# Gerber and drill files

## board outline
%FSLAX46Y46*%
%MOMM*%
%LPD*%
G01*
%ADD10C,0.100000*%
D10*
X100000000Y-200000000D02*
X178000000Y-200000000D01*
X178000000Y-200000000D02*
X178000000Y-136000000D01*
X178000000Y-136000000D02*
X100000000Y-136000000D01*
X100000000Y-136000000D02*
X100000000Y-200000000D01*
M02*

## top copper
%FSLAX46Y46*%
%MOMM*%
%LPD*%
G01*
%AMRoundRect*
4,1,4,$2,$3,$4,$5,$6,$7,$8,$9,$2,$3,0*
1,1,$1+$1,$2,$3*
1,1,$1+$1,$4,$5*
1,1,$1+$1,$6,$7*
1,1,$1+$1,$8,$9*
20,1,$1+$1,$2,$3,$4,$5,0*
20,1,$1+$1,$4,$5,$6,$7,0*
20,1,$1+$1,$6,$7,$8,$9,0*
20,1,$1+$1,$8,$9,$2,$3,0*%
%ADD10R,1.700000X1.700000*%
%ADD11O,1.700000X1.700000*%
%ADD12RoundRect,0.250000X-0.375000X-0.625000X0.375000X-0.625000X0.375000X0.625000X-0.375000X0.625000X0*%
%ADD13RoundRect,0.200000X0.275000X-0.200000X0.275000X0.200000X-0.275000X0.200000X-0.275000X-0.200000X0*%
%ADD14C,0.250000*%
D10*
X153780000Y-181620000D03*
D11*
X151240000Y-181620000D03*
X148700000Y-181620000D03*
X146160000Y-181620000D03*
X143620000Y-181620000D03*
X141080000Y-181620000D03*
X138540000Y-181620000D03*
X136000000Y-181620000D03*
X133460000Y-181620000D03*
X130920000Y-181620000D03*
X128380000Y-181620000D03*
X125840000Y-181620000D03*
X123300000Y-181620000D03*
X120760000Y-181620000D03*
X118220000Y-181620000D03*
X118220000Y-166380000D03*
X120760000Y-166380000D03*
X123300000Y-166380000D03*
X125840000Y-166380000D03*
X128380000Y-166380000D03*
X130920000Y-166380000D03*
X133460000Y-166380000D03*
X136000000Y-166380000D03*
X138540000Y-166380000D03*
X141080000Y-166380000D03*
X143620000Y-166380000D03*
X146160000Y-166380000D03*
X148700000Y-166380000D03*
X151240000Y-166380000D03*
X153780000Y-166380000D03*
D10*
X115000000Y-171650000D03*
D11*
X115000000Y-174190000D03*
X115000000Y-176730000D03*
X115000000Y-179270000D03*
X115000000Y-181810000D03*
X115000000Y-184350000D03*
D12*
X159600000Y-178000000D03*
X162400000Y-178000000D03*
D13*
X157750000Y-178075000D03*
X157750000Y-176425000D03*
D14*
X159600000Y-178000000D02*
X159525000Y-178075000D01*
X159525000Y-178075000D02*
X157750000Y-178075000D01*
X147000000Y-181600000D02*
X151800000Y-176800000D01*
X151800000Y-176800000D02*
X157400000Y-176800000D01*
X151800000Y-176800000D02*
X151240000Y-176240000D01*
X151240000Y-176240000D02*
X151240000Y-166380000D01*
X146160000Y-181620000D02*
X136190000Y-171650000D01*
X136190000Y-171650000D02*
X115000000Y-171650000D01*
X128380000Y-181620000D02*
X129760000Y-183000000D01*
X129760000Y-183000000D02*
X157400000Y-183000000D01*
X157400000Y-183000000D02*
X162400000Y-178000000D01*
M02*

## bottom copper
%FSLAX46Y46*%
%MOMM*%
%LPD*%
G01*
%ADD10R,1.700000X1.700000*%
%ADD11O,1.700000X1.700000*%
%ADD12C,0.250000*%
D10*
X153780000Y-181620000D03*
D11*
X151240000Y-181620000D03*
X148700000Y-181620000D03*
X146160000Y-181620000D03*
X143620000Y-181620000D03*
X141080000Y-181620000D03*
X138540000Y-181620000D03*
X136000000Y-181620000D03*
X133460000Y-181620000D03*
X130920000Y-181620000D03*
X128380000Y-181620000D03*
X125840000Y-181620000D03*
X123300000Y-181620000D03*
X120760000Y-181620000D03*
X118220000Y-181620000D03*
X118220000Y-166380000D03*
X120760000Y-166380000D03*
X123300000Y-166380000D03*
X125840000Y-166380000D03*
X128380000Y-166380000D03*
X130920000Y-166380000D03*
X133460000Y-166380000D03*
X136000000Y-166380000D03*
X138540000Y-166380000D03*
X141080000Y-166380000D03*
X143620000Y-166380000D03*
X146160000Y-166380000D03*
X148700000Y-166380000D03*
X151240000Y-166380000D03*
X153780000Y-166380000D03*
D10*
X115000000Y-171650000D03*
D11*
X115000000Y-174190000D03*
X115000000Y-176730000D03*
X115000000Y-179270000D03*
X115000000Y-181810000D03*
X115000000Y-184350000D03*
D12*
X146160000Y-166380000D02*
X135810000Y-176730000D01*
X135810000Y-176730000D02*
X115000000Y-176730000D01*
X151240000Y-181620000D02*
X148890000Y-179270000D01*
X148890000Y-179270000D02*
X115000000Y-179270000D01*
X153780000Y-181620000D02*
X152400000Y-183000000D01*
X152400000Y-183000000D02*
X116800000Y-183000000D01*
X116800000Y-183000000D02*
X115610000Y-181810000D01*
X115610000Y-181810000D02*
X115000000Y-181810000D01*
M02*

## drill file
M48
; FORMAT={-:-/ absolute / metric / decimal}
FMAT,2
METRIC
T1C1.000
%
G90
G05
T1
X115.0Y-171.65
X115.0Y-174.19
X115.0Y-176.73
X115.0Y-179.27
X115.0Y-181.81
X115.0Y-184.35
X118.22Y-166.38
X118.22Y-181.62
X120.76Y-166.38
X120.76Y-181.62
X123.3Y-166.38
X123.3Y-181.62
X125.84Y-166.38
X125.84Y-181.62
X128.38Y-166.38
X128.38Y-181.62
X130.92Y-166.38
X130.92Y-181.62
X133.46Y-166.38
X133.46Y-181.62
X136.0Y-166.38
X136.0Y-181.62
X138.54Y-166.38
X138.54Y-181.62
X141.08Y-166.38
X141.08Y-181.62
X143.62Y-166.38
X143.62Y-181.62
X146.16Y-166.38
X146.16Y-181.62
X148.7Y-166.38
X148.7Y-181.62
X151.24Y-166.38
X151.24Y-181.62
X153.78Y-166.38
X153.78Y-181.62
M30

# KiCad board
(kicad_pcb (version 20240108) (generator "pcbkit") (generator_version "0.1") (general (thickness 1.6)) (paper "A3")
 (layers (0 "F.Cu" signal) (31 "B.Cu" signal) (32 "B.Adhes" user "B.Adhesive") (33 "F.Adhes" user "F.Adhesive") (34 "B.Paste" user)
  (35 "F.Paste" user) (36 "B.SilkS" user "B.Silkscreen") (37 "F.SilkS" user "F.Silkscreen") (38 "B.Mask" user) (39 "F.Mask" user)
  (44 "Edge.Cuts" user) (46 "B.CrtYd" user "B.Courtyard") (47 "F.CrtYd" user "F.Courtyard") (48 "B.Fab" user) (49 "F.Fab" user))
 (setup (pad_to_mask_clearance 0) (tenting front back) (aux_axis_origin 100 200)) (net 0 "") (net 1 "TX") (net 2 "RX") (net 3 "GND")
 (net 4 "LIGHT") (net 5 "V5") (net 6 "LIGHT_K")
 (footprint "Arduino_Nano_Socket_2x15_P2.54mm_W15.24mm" (layer "B.Cu") (at 136 174 90)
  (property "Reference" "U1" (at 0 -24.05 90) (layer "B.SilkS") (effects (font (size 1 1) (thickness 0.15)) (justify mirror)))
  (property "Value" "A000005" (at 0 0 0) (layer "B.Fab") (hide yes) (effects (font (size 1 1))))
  (pad "1" thru_hole rect (at -7.62 17.78 90) (size 1.7 1.7) (drill 1) (layers "*.Cu" "*.Mask") (solder_mask_margin 0.05) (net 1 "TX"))
  (pad "2" thru_hole oval (at -7.62 15.24 90) (size 1.7 1.7) (drill 1) (layers "*.Cu" "*.Mask") (solder_mask_margin 0.05) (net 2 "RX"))
  (pad "3" thru_hole oval (at -7.62 12.7 90) (size 1.7 1.7) (drill 1) (layers "*.Cu" "*.Mask") (solder_mask_margin 0.05))
  (pad "4" thru_hole oval (at -7.62 10.16 90) (size 1.7 1.7) (drill 1) (layers "*.Cu" "*.Mask") (solder_mask_margin 0.05) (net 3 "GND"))
  (pad "5" thru_hole oval (at -7.62 7.62 90) (size 1.7 1.7) (drill 1) (layers "*.Cu" "*.Mask") (solder_mask_margin 0.05))
  (pad "6" thru_hole oval (at -7.62 5.08 90) (size 1.7 1.7) (drill 1) (layers "*.Cu" "*.Mask") (solder_mask_margin 0.05))
  (pad "7" thru_hole oval (at -7.62 2.54 90) (size 1.7 1.7) (drill 1) (layers "*.Cu" "*.Mask") (solder_mask_margin 0.05))
  (pad "8" thru_hole oval (at -7.62 0 90) (size 1.7 1.7) (drill 1) (layers "*.Cu" "*.Mask") (solder_mask_margin 0.05))
  (pad "9" thru_hole oval (at -7.62 -2.54 90) (size 1.7 1.7) (drill 1) (layers "*.Cu" "*.Mask") (solder_mask_margin 0.05))
  (pad "10" thru_hole oval (at -7.62 -5.08 90) (size 1.7 1.7) (drill 1) (layers "*.Cu" "*.Mask") (solder_mask_margin 0.05))
  (pad "11" thru_hole oval (at -7.62 -7.62 90) (size 1.7 1.7) (drill 1) (layers "*.Cu" "*.Mask") (solder_mask_margin 0.05) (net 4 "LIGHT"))
  (pad "12" thru_hole oval (at -7.62 -10.16 90) (size 1.7 1.7) (drill 1) (layers "*.Cu" "*.Mask") (solder_mask_margin 0.05))
  (pad "13" thru_hole oval (at -7.62 -12.7 90) (size 1.7 1.7) (drill 1) (layers "*.Cu" "*.Mask") (solder_mask_margin 0.05))
  (pad "14" thru_hole oval (at -7.62 -15.24 90) (size 1.7 1.7) (drill 1) (layers "*.Cu" "*.Mask") (solder_mask_margin 0.05))
  (pad "15" thru_hole oval (at -7.62 -17.78 90) (size 1.7 1.7) (drill 1) (layers "*.Cu" "*.Mask") (solder_mask_margin 0.05))
  (pad "16" thru_hole oval (at 7.62 -17.78 90) (size 1.7 1.7) (drill 1) (layers "*.Cu" "*.Mask") (solder_mask_margin 0.05))
  (pad "17" thru_hole oval (at 7.62 -15.24 90) (size 1.7 1.7) (drill 1) (layers "*.Cu" "*.Mask") (solder_mask_margin 0.05))
  (pad "18" thru_hole oval (at 7.62 -12.7 90) (size 1.7 1.7) (drill 1) (layers "*.Cu" "*.Mask") (solder_mask_margin 0.05))
  (pad "19" thru_hole oval (at 7.62 -10.16 90) (size 1.7 1.7) (drill 1) (layers "*.Cu" "*.Mask") (solder_mask_margin 0.05))
  (pad "20" thru_hole oval (at 7.62 -7.62 90) (size 1.7 1.7) (drill 1) (layers "*.Cu" "*.Mask") (solder_mask_margin 0.05))
  (pad "21" thru_hole oval (at 7.62 -5.08 90) (size 1.7 1.7) (drill 1) (layers "*.Cu" "*.Mask") (solder_mask_margin 0.05))
  (pad "22" thru_hole oval (at 7.62 -2.54 90) (size 1.7 1.7) (drill 1) (layers "*.Cu" "*.Mask") (solder_mask_margin 0.05))
  (pad "23" thru_hole oval (at 7.62 0 90) (size 1.7 1.7) (drill 1) (layers "*.Cu" "*.Mask") (solder_mask_margin 0.05))
  (pad "24" thru_hole oval (at 7.62 2.54 90) (size 1.7 1.7) (drill 1) (layers "*.Cu" "*.Mask") (solder_mask_margin 0.05))
  (pad "25" thru_hole oval (at 7.62 5.08 90) (size 1.7 1.7) (drill 1) (layers "*.Cu" "*.Mask") (solder_mask_margin 0.05))
  (pad "26" thru_hole oval (at 7.62 7.62 90) (size 1.7 1.7) (drill 1) (layers "*.Cu" "*.Mask") (solder_mask_margin 0.05))
  (pad "27" thru_hole oval (at 7.62 10.16 90) (size 1.7 1.7) (drill 1) (layers "*.Cu" "*.Mask") (solder_mask_margin 0.05) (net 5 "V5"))
  (pad "28" thru_hole oval (at 7.62 12.7 90) (size 1.7 1.7) (drill 1) (layers "*.Cu" "*.Mask") (solder_mask_margin 0.05))
  (pad "29" thru_hole oval (at 7.62 15.24 90) (size 1.7 1.7) (drill 1) (layers "*.Cu" "*.Mask") (solder_mask_margin 0.05) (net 3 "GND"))
  (pad "30" thru_hole oval (at 7.62 17.78 90) (size 1.7 1.7) (drill 1) (layers "*.Cu" "*.Mask") (solder_mask_margin 0.05)))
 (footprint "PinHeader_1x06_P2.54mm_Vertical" (layer "F.Cu") (at 115 178 0)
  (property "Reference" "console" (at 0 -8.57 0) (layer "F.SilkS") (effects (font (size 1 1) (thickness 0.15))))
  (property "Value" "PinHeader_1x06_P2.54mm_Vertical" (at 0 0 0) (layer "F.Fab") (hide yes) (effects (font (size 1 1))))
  (pad "1" thru_hole rect (at 0 -6.35 0) (size 1.7 1.7) (drill 1) (layers "*.Cu" "*.Mask") (solder_mask_margin 0.05) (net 3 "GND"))
  (pad "2" thru_hole oval (at 0 -3.81 0) (size 1.7 1.7) (drill 1) (layers "*.Cu" "*.Mask") (solder_mask_margin 0.05))
  (pad "3" thru_hole oval (at 0 -1.27 0) (size 1.7 1.7) (drill 1) (layers "*.Cu" "*.Mask") (solder_mask_margin 0.05) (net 5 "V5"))
  (pad "4" thru_hole oval (at 0 1.27 0) (size 1.7 1.7) (drill 1) (layers "*.Cu" "*.Mask") (solder_mask_margin 0.05) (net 2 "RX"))
  (pad "5" thru_hole oval (at 0 3.81 0) (size 1.7 1.7) (drill 1) (layers "*.Cu" "*.Mask") (solder_mask_margin 0.05) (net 1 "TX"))
  (pad "6" thru_hole oval (at 0 6.35 0) (size 1.7 1.7) (drill 1) (layers "*.Cu" "*.Mask") (solder_mask_margin 0.05)))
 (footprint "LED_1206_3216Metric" (layer "F.Cu") (at 161 178 0)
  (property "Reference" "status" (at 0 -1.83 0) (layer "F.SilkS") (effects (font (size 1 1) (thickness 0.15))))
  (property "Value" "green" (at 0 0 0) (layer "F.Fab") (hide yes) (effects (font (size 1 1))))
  (pad "1" smd roundrect (at -1.4 0 0) (size 1.25 1.75) (layers "F.Cu" "F.Paste" "F.Mask") (roundrect_rratio 0.200000000000)
   (solder_mask_margin 0.05) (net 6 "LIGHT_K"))
  (pad "2" smd roundrect (at 1.4 0 0) (size 1.25 1.75) (layers "F.Cu" "F.Paste" "F.Mask") (roundrect_rratio 0.200000000000)
   (solder_mask_margin 0.05) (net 4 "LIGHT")))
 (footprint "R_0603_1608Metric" (layer "F.Cu") (at 157.75 177.25 90)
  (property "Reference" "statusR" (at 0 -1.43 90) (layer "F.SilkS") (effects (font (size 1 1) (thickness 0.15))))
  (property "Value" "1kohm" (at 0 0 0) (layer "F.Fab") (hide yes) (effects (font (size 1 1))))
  (pad "1" smd roundrect (at -0.825 0 90) (size 0.8 0.95) (layers "F.Cu" "F.Paste" "F.Mask") (roundrect_rratio 0.250000000000)
   (solder_mask_margin 0.05) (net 6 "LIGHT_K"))
  (pad "2" smd roundrect (at 0.825 0 90) (size 0.8 0.95) (layers "F.Cu" "F.Paste" "F.Mask") (roundrect_rratio 0.250000000000)
   (solder_mask_margin 0.05) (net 3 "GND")))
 (segment (start 159.6 178) (end 159.525 178.075) (width 0.25) (layer "F.Cu") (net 6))
 (segment (start 159.525 178.075) (end 157.75 178.075) (width 0.25) (layer "F.Cu") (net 6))
 (segment (start 147 181.6) (end 151.8 176.8) (width 0.25) (layer "F.Cu") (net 3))
 (segment (start 151.8 176.8) (end 157.4 176.8) (width 0.25) (layer "F.Cu") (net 3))
 (segment (start 151.8 176.8) (end 151.24 176.24) (width 0.25) (layer "F.Cu") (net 3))
 (segment (start 151.24 176.24) (end 151.24 166.38) (width 0.25) (layer "F.Cu") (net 3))
 (segment (start 146.16 181.62) (end 136.19 171.65) (width 0.25) (layer "F.Cu") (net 3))
 (segment (start 136.19 171.65) (end 115 171.65) (width 0.25) (layer "F.Cu") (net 3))
 (segment (start 146.16 166.38) (end 135.81 176.73) (width 0.25) (layer "B.Cu") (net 5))
 (segment (start 135.81 176.73) (end 115 176.73) (width 0.25) (layer "B.Cu") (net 5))
 (segment (start 151.24 181.62) (end 148.89 179.27) (width 0.25) (layer "B.Cu") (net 2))
 (segment (start 148.89 179.27) (end 115 179.27) (width 0.25) (layer "B.Cu") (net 2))
 (segment (start 128.38 181.62) (end 129.76 183) (width 0.25) (layer "F.Cu") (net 4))
 (segment (start 129.76 183) (end 157.4 183) (width 0.25) (layer "F.Cu") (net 4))
 (segment (start 157.4 183) (end 162.4 178) (width 0.25) (layer "F.Cu") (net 4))
 (segment (start 153.78 181.62) (end 152.4 183) (width 0.25) (layer "B.Cu") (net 1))
 (segment (start 152.4 183) (end 116.8 183) (width 0.25) (layer "B.Cu") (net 1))
 (segment (start 116.8 183) (end 115.61 181.81) (width 0.25) (layer "B.Cu") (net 1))
 (segment (start 115.61 181.81) (end 115 181.81) (width 0.25) (layer "B.Cu") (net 1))
 (gr_line (start 100 200) (end 178 200) (stroke (width 0.1) (type solid)) (layer "Edge.Cuts"))
 (gr_line (start 178 200) (end 178 136) (stroke (width 0.1) (type solid)) (layer "Edge.Cuts"))
 (gr_line (start 178 136) (end 100 136) (stroke (width 0.1) (type solid)) (layer "Edge.Cuts"))
 (gr_line (start 100 136) (end 100 200) (stroke (width 0.1) (type solid)) (layer "Edge.Cuts")))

